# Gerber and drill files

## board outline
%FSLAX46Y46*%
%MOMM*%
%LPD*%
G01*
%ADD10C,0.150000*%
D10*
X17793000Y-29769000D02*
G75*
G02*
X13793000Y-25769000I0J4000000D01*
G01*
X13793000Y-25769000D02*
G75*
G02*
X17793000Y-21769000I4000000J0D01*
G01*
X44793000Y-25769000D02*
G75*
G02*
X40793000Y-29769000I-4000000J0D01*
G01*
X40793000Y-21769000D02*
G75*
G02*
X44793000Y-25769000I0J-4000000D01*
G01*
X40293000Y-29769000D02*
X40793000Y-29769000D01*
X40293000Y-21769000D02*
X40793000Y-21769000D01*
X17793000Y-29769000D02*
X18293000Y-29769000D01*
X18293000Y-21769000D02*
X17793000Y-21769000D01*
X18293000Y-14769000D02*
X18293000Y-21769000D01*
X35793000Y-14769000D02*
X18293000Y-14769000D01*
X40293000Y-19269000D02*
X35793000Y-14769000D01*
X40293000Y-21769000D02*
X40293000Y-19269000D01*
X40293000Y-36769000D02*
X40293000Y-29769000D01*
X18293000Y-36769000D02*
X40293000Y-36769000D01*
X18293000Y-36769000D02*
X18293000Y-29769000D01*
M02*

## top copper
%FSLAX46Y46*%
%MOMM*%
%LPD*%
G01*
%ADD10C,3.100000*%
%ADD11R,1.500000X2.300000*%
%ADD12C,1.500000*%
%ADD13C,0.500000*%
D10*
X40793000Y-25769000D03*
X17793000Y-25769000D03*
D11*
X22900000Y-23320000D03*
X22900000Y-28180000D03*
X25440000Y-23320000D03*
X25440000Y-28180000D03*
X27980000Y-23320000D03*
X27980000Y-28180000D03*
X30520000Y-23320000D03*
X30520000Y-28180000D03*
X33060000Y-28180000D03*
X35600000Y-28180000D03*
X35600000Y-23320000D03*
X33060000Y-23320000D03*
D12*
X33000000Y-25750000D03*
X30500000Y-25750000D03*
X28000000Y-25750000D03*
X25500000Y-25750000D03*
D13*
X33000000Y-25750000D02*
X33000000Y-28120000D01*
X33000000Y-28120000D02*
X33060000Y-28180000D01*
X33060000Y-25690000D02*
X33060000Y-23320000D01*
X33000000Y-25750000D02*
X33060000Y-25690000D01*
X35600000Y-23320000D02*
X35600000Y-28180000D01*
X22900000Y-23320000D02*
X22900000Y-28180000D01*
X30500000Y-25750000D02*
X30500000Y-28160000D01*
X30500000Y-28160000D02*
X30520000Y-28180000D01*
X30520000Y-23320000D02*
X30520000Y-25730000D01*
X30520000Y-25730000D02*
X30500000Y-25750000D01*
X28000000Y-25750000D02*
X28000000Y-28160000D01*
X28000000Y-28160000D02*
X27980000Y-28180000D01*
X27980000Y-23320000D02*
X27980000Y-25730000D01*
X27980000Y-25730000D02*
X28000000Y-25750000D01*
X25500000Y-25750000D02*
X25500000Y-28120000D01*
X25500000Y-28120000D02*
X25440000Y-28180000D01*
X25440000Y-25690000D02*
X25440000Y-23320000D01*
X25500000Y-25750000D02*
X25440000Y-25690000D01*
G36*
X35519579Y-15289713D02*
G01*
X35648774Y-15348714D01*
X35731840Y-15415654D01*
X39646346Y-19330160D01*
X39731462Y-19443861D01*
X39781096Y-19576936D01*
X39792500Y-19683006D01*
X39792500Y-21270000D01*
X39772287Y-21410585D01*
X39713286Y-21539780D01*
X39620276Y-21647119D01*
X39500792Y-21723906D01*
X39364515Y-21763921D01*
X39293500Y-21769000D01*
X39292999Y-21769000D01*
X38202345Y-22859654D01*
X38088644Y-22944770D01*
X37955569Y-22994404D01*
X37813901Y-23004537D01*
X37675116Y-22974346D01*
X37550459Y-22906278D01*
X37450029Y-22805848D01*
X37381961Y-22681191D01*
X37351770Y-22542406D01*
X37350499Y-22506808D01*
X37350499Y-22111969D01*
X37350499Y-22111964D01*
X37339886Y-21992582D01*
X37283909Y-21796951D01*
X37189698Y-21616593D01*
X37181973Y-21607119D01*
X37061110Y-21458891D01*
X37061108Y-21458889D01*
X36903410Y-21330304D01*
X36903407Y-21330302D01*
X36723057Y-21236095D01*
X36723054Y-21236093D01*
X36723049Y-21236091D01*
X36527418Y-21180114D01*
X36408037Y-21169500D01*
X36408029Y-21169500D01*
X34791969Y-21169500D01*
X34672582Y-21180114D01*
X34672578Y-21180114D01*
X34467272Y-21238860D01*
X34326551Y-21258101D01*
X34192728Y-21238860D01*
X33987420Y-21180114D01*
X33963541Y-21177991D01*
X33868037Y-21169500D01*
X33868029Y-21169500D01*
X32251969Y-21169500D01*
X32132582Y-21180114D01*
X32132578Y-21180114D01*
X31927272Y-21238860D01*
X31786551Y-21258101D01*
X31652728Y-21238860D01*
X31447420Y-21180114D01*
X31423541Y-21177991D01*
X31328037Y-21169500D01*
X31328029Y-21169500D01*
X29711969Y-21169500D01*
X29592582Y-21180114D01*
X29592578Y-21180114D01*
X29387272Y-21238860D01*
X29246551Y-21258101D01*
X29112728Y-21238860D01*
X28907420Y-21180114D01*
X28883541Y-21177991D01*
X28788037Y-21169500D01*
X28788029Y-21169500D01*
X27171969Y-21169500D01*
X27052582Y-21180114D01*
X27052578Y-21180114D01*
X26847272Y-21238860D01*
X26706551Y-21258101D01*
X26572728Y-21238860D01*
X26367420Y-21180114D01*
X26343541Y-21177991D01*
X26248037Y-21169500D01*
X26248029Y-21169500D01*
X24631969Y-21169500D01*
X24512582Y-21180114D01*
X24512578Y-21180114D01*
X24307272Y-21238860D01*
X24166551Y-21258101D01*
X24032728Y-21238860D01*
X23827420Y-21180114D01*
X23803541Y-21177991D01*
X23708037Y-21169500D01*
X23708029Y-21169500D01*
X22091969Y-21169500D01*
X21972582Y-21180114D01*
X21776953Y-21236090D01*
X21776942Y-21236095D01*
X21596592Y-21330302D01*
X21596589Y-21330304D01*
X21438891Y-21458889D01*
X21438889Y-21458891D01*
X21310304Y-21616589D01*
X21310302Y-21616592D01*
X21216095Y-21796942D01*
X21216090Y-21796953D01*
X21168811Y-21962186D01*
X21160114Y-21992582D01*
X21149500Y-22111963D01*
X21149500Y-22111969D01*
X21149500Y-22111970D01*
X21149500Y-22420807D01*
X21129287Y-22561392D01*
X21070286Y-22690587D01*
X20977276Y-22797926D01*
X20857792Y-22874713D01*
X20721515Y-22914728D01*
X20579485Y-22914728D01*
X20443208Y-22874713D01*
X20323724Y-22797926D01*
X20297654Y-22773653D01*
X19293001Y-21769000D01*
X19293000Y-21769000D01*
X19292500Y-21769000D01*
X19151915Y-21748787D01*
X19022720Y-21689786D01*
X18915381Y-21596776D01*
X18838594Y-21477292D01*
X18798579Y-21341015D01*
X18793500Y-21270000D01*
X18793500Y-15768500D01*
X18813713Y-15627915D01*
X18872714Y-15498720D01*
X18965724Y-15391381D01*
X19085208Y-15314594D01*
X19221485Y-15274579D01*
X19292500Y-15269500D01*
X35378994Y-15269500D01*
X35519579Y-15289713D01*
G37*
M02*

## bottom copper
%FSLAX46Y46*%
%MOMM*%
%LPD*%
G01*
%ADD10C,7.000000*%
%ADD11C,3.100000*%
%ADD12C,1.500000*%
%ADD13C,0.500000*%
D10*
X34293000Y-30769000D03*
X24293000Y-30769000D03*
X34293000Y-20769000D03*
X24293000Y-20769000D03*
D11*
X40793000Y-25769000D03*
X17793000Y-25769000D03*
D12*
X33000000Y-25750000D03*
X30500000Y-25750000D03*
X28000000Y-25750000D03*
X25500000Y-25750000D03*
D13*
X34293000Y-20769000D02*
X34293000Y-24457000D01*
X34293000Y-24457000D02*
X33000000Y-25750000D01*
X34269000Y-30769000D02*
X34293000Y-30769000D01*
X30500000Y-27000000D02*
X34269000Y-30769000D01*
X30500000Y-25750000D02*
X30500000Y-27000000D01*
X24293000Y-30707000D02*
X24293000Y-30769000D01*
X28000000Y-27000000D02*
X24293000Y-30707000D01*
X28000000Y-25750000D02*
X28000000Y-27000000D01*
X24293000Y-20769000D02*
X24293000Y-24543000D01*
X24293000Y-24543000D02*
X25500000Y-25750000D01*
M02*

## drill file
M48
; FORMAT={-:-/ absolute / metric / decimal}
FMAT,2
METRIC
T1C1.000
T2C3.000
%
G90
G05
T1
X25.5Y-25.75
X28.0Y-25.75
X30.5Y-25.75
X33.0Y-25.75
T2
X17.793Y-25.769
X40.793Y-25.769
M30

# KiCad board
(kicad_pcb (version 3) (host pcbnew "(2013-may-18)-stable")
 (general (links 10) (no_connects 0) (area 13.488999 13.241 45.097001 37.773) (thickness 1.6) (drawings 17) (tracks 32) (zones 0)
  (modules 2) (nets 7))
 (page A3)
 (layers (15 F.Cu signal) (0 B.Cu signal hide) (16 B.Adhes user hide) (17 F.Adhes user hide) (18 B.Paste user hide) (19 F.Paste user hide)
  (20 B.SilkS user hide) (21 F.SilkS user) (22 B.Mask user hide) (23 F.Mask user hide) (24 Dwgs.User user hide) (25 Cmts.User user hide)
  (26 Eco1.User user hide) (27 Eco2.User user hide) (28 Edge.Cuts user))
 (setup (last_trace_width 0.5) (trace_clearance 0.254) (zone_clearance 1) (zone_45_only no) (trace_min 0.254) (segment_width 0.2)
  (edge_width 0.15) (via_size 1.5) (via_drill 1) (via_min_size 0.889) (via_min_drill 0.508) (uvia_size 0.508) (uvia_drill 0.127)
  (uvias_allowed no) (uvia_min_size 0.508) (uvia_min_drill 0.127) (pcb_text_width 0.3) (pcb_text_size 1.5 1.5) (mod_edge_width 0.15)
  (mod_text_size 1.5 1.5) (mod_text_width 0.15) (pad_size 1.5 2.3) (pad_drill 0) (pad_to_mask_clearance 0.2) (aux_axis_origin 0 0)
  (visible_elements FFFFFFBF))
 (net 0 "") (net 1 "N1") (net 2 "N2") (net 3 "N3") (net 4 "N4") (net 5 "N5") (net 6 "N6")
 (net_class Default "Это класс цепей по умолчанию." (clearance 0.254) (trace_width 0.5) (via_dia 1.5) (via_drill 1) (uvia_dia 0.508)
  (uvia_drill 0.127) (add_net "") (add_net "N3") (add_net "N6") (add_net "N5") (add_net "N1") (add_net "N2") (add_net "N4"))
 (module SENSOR (layer B.Cu) (at 40.793 37.269 180)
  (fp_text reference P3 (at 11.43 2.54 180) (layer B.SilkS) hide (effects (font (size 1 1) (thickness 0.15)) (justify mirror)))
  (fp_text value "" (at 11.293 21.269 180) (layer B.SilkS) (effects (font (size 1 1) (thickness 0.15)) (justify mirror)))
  (pad 2 smd circle (at 6.5 6.5 180) (size 7 7) (layers B.Cu B.Mask) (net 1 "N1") (solder_mask_margin 0.1))
  (pad 3 smd circle (at 16.5 6.5 180) (size 7 7) (layers B.Cu B.Mask) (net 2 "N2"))
  (pad 1 smd circle (at 6.5 16.5 180) (size 7 7) (layers B.Cu B.Mask) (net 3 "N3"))
  (pad 4 smd circle (at 16.5 16.5 180) (size 7 7) (layers B.Cu B.Mask) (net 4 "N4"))
  (pad "" np_thru_hole circle (at 0 11.5 180) (size 3.1 3.1) (drill 3) (layers *.Cu *.Mask B.SilkS))
  (pad "" np_thru_hole circle (at 23 11.5 180) (size 3.1 3.1) (drill 3) (layers *.Cu *.Mask B.SilkS)))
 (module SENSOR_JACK (layer F.Cu) (at 29.25 25.75)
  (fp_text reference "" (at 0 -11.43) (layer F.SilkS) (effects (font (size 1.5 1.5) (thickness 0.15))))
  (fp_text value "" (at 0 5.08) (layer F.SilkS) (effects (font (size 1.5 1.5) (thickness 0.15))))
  (pad 12 smd rect (at -6.35 -2.43) (size 1.5 2.3) (layers F.Cu F.Paste F.Mask) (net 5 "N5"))
  (pad 1 smd rect (at -6.35 2.43) (size 1.5 2.3) (layers F.Cu F.Paste F.Mask) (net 5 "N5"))
  (pad 11 smd rect (at -3.81 -2.43) (size 1.5 2.3) (layers F.Cu F.Paste F.Mask) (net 4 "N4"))
  (pad 2 smd rect (at -3.81 2.43) (size 1.5 2.3) (layers F.Cu F.Paste F.Mask) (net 4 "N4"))
  (pad 10 smd rect (at -1.27 -2.43) (size 1.5 2.3) (layers F.Cu F.Paste F.Mask) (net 2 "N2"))
  (pad 3 smd rect (at -1.27 2.43) (size 1.5 2.3) (layers F.Cu F.Paste F.Mask) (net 2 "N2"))
  (pad 9 smd rect (at 1.27 -2.43) (size 1.5 2.3) (layers F.Cu F.Paste F.Mask) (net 1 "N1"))
  (pad 4 smd rect (at 1.27 2.43) (size 1.5 2.3) (layers F.Cu F.Paste F.Mask) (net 1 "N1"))
  (pad 5 smd rect (at 3.81 2.43) (size 1.5 2.3) (layers F.Cu F.Paste F.Mask) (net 3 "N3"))
  (pad 6 smd rect (at 6.35 2.43) (size 1.5 2.3) (layers F.Cu F.Paste F.Mask) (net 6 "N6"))
  (pad 7 smd rect (at 6.35 -2.43) (size 1.5 2.3) (layers F.Cu F.Paste F.Mask) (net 6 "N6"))
  (pad 8 smd rect (at 3.81 -2.43) (size 1.5 2.3) (layers F.Cu F.Paste F.Mask) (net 3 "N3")))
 (gr_arc (start 17.793 25.769) (end 17.793 29.769) (angle 90) (layer Edge.Cuts) (width 0.15))
 (gr_arc (start 17.793 25.769) (end 13.793 25.769) (angle 90) (layer Edge.Cuts) (width 0.15))
 (gr_arc (start 40.793 25.769) (end 44.793 25.769) (angle 90) (layer Edge.Cuts) (width 0.15))
 (gr_arc (start 40.793 25.769) (end 40.793 21.769) (angle 90) (layer Edge.Cuts) (width 0.15))
 (gr_line (start 40.293 29.769) (end 40.793 29.769) (angle 90) (layer Edge.Cuts) (width 0.15))
 (gr_line (start 40.293 21.769) (end 40.793 21.769) (angle 90) (layer Edge.Cuts) (width 0.15))
 (gr_line (start 17.793 29.769) (end 18.293 29.769) (angle 90) (layer Edge.Cuts) (width 0.15))
 (gr_line (start 18.293 21.769) (end 17.793 21.769) (angle 90) (layer Edge.Cuts) (width 0.15))
 (gr_line (start 18.293 14.769) (end 18.293 21.769) (angle 90) (layer Edge.Cuts) (width 0.15))
 (gr_line (start 35.793 14.769) (end 18.293 14.769) (angle 90) (layer Edge.Cuts) (width 0.15))
 (gr_line (start 40.293 19.269) (end 35.793 14.769) (angle 90) (layer Edge.Cuts) (width 0.15))
 (gr_line (start 40.293 21.769) (end 40.293 19.269) (angle 90) (layer Edge.Cuts) (width 0.15))
 (gr_line (start 40.293 36.769) (end 40.293 29.769) (angle 90) (layer Edge.Cuts) (width 0.15))
 (gr_line (start 18.293 36.769) (end 40.293 36.769) (angle 90) (layer Edge.Cuts) (width 0.15))
 (gr_line (start 18.293 36.769) (end 18.293 29.769) (angle 90) (layer Edge.Cuts) (width 0.15))
 (segment (start 33 25.75) (end 33 28.12) (width 0.5) (layer F.Cu) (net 3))
 (segment (start 33 28.12) (end 33.06 28.18) (width 0.5) (layer F.Cu) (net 3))
 (segment (start 34.293 20.769) (end 34.293 24.457) (width 0.5) (layer B.Cu) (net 3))
 (segment (start 33.06 25.69) (end 33.06 23.32) (width 0.5) (layer F.Cu) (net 3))
 (segment (start 33 25.75) (end 33.06 25.69) (width 0.5) (layer F.Cu) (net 3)) (via (at 33 25.75) (size 1.5) (layers F.Cu B.Cu) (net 3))
 (segment (start 34.293 24.457) (end 33 25.75) (width 0.5) (layer B.Cu) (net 3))
 (segment (start 35.6 23.32) (end 35.6 28.18) (width 0.5) (layer F.Cu) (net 6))
 (segment (start 22.9 23.32) (end 22.9 28.18) (width 0.5) (layer F.Cu) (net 5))
 (segment (start 30.5 25.75) (end 30.5 28.16) (width 0.5) (layer F.Cu) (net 1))
 (segment (start 30.5 28.16) (end 30.52 28.18) (width 0.5) (layer F.Cu) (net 1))
 (segment (start 30.52 23.32) (end 30.52 25.73) (width 0.5) (layer F.Cu) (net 1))
 (segment (start 34.269 30.769) (end 34.293 30.769) (width 0.5) (layer B.Cu) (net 1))
 (segment (start 30.5 27) (end 34.269 30.769) (width 0.5) (layer B.Cu) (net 1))
 (segment (start 30.5 25.75) (end 30.5 27) (width 0.5) (layer B.Cu) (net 1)) (via (at 30.5 25.75) (size 1.5) (layers F.Cu B.Cu) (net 1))
 (segment (start 30.52 25.73) (end 30.5 25.75) (width 0.5) (layer F.Cu) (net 1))
 (segment (start 28 25.75) (end 28 28.16) (width 0.5) (layer F.Cu) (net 2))
 (segment (start 28 28.16) (end 27.98 28.18) (width 0.5) (layer F.Cu) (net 2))
 (segment (start 27.98 23.32) (end 27.98 25.73) (width 0.5) (layer F.Cu) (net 2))
 (segment (start 24.293 30.707) (end 24.293 30.769) (width 0.5) (layer B.Cu) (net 2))
 (segment (start 28 27) (end 24.293 30.707) (width 0.5) (layer B.Cu) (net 2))
 (segment (start 28 25.75) (end 28 27) (width 0.5) (layer B.Cu) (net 2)) (via (at 28 25.75) (size 1.5) (layers F.Cu B.Cu) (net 2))
 (segment (start 27.98 25.73) (end 28 25.75) (width 0.5) (layer F.Cu) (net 2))
 (segment (start 25.5 25.75) (end 25.5 28.12) (width 0.5) (layer F.Cu) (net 4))
 (segment (start 25.5 28.12) (end 25.44 28.18) (width 0.5) (layer F.Cu) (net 4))
 (segment (start 24.293 20.769) (end 24.293 24.543) (width 0.5) (layer B.Cu) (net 4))
 (segment (start 25.44 25.69) (end 25.44 23.32) (width 0.5) (layer F.Cu) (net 4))
 (segment (start 25.5 25.75) (end 25.44 25.69) (width 0.5) (layer F.Cu) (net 4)) (via (at 25.5 25.75) (size 1.5) (layers F.Cu B.Cu) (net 4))
 (segment (start 24.293 24.543) (end 25.5 25.75) (width 0.5) (layer B.Cu) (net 4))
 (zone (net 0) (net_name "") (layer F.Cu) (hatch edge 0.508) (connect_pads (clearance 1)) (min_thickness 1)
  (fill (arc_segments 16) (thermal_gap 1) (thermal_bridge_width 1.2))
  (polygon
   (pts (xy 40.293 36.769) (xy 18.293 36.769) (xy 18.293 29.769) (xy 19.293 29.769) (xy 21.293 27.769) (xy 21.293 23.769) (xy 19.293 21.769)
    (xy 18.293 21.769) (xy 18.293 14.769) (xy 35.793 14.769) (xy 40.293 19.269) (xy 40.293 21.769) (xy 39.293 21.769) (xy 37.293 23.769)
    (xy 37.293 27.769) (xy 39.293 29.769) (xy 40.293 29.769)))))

